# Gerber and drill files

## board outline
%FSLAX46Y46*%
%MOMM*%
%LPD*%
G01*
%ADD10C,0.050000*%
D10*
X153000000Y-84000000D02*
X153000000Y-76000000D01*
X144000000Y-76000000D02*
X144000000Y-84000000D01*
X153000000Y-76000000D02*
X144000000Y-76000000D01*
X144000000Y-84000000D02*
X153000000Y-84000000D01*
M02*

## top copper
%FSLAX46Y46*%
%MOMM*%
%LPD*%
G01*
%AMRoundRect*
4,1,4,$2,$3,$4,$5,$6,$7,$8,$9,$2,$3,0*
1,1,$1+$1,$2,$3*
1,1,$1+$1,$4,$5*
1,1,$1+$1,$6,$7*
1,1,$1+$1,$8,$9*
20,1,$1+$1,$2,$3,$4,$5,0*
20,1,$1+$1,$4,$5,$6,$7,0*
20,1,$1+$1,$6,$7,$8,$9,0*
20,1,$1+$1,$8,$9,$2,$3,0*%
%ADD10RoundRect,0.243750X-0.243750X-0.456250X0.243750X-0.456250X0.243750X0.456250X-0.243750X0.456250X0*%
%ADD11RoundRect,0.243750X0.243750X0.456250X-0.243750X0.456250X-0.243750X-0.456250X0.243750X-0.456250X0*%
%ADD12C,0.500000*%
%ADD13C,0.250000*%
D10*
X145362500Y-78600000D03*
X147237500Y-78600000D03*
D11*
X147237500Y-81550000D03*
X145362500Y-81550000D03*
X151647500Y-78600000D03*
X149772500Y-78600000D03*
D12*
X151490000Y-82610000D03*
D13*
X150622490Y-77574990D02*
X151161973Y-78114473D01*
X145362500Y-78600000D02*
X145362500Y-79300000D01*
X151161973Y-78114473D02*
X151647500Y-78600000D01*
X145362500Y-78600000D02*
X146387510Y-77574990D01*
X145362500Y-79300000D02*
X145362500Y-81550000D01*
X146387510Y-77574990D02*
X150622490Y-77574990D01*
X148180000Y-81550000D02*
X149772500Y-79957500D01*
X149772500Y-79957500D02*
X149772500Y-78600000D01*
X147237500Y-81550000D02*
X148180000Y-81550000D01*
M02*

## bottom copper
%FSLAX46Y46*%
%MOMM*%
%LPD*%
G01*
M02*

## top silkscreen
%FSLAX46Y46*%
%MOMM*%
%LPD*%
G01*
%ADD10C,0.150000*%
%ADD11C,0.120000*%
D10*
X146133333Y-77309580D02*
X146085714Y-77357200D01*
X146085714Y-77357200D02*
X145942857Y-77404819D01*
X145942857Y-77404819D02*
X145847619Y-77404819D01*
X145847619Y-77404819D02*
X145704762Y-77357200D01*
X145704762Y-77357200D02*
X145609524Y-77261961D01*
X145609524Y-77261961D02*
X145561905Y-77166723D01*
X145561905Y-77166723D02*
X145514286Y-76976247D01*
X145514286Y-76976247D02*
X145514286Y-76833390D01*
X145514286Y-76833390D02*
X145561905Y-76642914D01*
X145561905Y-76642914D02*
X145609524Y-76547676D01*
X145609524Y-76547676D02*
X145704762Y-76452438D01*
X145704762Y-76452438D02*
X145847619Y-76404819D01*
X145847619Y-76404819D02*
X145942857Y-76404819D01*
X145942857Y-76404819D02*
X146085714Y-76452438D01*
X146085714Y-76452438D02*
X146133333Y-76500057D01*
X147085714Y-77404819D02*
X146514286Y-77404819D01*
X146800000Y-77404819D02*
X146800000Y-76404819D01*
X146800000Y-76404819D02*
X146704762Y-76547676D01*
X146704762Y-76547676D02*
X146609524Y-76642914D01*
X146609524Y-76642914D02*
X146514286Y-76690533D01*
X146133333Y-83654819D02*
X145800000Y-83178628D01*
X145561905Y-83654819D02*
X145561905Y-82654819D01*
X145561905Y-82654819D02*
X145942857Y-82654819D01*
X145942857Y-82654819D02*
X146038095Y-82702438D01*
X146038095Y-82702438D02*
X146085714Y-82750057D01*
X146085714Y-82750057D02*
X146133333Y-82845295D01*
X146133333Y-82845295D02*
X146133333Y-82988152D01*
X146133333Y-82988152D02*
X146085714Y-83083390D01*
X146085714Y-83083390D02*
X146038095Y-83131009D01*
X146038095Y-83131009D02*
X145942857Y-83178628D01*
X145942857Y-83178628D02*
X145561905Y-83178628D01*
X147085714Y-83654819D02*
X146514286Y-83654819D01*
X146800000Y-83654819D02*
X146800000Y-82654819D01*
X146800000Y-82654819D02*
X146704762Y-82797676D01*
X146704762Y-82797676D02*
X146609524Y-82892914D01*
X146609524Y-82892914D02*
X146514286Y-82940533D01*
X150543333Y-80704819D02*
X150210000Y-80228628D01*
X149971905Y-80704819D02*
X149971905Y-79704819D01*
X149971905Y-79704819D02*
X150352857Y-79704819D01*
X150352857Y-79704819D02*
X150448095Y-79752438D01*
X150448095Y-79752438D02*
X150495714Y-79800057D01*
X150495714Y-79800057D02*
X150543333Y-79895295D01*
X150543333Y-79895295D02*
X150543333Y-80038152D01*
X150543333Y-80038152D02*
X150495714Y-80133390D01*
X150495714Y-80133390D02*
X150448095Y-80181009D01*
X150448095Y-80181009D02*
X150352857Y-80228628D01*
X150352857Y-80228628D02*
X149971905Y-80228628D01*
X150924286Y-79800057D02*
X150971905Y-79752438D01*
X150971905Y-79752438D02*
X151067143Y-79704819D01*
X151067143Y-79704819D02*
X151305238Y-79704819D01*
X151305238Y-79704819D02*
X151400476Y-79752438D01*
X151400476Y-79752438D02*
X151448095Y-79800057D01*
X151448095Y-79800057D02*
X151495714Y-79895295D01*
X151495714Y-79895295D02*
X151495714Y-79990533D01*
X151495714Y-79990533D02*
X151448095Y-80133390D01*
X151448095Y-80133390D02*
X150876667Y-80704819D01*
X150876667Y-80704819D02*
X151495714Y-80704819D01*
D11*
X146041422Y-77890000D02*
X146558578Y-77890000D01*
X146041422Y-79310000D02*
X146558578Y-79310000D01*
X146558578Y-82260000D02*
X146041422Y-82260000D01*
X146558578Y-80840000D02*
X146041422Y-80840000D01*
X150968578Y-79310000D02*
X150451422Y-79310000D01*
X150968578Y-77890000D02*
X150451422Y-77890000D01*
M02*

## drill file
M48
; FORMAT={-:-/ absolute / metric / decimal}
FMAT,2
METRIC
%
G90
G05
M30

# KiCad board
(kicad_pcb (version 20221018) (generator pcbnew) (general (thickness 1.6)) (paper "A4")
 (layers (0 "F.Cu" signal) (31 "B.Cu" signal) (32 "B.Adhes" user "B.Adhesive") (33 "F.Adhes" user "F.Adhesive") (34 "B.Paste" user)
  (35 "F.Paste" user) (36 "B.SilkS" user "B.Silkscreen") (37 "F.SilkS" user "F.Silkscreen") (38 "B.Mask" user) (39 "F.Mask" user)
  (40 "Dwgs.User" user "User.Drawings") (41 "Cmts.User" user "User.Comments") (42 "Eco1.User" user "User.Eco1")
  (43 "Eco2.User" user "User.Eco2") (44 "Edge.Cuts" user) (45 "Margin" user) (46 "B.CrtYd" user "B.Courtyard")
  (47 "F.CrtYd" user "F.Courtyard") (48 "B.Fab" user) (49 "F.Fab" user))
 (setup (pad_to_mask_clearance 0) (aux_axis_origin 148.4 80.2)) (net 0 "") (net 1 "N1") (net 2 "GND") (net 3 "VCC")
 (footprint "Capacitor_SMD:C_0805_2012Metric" (layer "F.Cu") (at 146.3 78.6)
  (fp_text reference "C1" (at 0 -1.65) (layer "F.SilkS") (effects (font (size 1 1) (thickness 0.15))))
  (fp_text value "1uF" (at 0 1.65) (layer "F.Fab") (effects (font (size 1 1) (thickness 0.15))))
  (fp_line (start -0.258578 -0.71) (end 0.258578 -0.71) (stroke (width 0.12) (type solid)) (layer "F.SilkS"))
  (fp_line (start -0.258578 0.71) (end 0.258578 0.71) (stroke (width 0.12) (type solid)) (layer "F.SilkS"))
  (pad "1" smd roundrect (at -0.9375 0) (size 0.975 1.4) (layers "F.Cu" "F.Paste" "F.Mask") (roundrect_rratio 0.25) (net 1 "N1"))
  (pad "2" smd roundrect (at 0.9375 0) (size 0.975 1.4) (layers "F.Cu" "F.Paste" "F.Mask") (roundrect_rratio 0.25) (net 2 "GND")))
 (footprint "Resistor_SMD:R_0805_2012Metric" (layer "F.Cu") (at 146.3 81.55 180)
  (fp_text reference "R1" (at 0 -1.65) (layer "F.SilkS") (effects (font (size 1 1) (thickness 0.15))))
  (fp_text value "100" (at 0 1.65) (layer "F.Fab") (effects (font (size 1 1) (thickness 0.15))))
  (fp_line (start -0.258578 -0.71) (end 0.258578 -0.71) (stroke (width 0.12) (type solid)) (layer "F.SilkS"))
  (fp_line (start -0.258578 0.71) (end 0.258578 0.71) (stroke (width 0.12) (type solid)) (layer "F.SilkS"))
  (pad "1" smd roundrect (at -0.9375 0 180) (size 0.975 1.4) (layers "F.Cu" "F.Paste" "F.Mask") (roundrect_rratio 0.25) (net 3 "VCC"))
  (pad "2" smd roundrect (at 0.9375 0 180) (size 0.975 1.4) (layers "F.Cu" "F.Paste" "F.Mask") (roundrect_rratio 0.25) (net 1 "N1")))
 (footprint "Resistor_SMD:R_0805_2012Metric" (layer "F.Cu") (at 150.71 78.6 180)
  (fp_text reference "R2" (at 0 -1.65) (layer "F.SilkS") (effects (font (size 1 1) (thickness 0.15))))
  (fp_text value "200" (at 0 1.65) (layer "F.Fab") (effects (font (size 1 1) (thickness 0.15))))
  (fp_line (start -0.258578 -0.71) (end 0.258578 -0.71) (stroke (width 0.12) (type solid)) (layer "F.SilkS"))
  (fp_line (start -0.258578 0.71) (end 0.258578 0.71) (stroke (width 0.12) (type solid)) (layer "F.SilkS"))
  (pad "1" smd roundrect (at -0.9375 0 180) (size 0.975 1.4) (layers "F.Cu" "F.Paste" "F.Mask") (roundrect_rratio 0.25) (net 1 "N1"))
  (pad "2" smd roundrect (at 0.9375 0 180) (size 0.975 1.4) (layers "F.Cu" "F.Paste" "F.Mask") (roundrect_rratio 0.25) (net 3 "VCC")))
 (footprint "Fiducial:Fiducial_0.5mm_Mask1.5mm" (layer "F.Cu") (at 151.49 82.61)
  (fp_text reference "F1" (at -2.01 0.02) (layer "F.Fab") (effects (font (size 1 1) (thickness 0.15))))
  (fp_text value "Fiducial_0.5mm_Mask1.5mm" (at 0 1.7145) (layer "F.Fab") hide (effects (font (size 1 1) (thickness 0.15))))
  (pad "" smd circle (at 0 0) (size 0.5 0.5) (layers "F.Cu" "F.Mask") (solder_mask_margin 0.5) (clearance 0.5)))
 (gr_line (start 153 84) (end 153 76) (stroke (width 0.05) (type solid)) (layer "Edge.Cuts"))
 (gr_line (start 144 76) (end 144 84) (stroke (width 0.05) (type solid)) (layer "Edge.Cuts"))
 (gr_line (start 153 76) (end 144 76) (stroke (width 0.05) (type solid)) (layer "Edge.Cuts"))
 (gr_line (start 144 84) (end 153 84) (stroke (width 0.05) (type solid)) (layer "Edge.Cuts"))
 (segment (start 150.62249 77.57499) (end 151.161973 78.114473) (width 0.25) (layer "F.Cu") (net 1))
 (segment (start 145.3625 78.6) (end 145.3625 79.3) (width 0.25) (layer "F.Cu") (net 1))
 (segment (start 151.161973 78.114473) (end 151.6475 78.6) (width 0.25) (layer "F.Cu") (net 1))
 (segment (start 145.3625 78.6) (end 146.38751 77.57499) (width 0.25) (layer "F.Cu") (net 1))
 (segment (start 145.3625 79.3) (end 145.3625 81.55) (width 0.25) (layer "F.Cu") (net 1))
 (segment (start 146.38751 77.57499) (end 150.62249 77.57499) (width 0.25) (layer "F.Cu") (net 1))
 (segment (start 148.18 81.55) (end 149.7725 79.9575) (width 0.25) (layer "F.Cu") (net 3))
 (segment (start 149.7725 79.9575) (end 149.7725 78.6) (width 0.25) (layer "F.Cu") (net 3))
 (segment (start 147.2375 81.55) (end 148.18 81.55) (width 0.25) (layer "F.Cu") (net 3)))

